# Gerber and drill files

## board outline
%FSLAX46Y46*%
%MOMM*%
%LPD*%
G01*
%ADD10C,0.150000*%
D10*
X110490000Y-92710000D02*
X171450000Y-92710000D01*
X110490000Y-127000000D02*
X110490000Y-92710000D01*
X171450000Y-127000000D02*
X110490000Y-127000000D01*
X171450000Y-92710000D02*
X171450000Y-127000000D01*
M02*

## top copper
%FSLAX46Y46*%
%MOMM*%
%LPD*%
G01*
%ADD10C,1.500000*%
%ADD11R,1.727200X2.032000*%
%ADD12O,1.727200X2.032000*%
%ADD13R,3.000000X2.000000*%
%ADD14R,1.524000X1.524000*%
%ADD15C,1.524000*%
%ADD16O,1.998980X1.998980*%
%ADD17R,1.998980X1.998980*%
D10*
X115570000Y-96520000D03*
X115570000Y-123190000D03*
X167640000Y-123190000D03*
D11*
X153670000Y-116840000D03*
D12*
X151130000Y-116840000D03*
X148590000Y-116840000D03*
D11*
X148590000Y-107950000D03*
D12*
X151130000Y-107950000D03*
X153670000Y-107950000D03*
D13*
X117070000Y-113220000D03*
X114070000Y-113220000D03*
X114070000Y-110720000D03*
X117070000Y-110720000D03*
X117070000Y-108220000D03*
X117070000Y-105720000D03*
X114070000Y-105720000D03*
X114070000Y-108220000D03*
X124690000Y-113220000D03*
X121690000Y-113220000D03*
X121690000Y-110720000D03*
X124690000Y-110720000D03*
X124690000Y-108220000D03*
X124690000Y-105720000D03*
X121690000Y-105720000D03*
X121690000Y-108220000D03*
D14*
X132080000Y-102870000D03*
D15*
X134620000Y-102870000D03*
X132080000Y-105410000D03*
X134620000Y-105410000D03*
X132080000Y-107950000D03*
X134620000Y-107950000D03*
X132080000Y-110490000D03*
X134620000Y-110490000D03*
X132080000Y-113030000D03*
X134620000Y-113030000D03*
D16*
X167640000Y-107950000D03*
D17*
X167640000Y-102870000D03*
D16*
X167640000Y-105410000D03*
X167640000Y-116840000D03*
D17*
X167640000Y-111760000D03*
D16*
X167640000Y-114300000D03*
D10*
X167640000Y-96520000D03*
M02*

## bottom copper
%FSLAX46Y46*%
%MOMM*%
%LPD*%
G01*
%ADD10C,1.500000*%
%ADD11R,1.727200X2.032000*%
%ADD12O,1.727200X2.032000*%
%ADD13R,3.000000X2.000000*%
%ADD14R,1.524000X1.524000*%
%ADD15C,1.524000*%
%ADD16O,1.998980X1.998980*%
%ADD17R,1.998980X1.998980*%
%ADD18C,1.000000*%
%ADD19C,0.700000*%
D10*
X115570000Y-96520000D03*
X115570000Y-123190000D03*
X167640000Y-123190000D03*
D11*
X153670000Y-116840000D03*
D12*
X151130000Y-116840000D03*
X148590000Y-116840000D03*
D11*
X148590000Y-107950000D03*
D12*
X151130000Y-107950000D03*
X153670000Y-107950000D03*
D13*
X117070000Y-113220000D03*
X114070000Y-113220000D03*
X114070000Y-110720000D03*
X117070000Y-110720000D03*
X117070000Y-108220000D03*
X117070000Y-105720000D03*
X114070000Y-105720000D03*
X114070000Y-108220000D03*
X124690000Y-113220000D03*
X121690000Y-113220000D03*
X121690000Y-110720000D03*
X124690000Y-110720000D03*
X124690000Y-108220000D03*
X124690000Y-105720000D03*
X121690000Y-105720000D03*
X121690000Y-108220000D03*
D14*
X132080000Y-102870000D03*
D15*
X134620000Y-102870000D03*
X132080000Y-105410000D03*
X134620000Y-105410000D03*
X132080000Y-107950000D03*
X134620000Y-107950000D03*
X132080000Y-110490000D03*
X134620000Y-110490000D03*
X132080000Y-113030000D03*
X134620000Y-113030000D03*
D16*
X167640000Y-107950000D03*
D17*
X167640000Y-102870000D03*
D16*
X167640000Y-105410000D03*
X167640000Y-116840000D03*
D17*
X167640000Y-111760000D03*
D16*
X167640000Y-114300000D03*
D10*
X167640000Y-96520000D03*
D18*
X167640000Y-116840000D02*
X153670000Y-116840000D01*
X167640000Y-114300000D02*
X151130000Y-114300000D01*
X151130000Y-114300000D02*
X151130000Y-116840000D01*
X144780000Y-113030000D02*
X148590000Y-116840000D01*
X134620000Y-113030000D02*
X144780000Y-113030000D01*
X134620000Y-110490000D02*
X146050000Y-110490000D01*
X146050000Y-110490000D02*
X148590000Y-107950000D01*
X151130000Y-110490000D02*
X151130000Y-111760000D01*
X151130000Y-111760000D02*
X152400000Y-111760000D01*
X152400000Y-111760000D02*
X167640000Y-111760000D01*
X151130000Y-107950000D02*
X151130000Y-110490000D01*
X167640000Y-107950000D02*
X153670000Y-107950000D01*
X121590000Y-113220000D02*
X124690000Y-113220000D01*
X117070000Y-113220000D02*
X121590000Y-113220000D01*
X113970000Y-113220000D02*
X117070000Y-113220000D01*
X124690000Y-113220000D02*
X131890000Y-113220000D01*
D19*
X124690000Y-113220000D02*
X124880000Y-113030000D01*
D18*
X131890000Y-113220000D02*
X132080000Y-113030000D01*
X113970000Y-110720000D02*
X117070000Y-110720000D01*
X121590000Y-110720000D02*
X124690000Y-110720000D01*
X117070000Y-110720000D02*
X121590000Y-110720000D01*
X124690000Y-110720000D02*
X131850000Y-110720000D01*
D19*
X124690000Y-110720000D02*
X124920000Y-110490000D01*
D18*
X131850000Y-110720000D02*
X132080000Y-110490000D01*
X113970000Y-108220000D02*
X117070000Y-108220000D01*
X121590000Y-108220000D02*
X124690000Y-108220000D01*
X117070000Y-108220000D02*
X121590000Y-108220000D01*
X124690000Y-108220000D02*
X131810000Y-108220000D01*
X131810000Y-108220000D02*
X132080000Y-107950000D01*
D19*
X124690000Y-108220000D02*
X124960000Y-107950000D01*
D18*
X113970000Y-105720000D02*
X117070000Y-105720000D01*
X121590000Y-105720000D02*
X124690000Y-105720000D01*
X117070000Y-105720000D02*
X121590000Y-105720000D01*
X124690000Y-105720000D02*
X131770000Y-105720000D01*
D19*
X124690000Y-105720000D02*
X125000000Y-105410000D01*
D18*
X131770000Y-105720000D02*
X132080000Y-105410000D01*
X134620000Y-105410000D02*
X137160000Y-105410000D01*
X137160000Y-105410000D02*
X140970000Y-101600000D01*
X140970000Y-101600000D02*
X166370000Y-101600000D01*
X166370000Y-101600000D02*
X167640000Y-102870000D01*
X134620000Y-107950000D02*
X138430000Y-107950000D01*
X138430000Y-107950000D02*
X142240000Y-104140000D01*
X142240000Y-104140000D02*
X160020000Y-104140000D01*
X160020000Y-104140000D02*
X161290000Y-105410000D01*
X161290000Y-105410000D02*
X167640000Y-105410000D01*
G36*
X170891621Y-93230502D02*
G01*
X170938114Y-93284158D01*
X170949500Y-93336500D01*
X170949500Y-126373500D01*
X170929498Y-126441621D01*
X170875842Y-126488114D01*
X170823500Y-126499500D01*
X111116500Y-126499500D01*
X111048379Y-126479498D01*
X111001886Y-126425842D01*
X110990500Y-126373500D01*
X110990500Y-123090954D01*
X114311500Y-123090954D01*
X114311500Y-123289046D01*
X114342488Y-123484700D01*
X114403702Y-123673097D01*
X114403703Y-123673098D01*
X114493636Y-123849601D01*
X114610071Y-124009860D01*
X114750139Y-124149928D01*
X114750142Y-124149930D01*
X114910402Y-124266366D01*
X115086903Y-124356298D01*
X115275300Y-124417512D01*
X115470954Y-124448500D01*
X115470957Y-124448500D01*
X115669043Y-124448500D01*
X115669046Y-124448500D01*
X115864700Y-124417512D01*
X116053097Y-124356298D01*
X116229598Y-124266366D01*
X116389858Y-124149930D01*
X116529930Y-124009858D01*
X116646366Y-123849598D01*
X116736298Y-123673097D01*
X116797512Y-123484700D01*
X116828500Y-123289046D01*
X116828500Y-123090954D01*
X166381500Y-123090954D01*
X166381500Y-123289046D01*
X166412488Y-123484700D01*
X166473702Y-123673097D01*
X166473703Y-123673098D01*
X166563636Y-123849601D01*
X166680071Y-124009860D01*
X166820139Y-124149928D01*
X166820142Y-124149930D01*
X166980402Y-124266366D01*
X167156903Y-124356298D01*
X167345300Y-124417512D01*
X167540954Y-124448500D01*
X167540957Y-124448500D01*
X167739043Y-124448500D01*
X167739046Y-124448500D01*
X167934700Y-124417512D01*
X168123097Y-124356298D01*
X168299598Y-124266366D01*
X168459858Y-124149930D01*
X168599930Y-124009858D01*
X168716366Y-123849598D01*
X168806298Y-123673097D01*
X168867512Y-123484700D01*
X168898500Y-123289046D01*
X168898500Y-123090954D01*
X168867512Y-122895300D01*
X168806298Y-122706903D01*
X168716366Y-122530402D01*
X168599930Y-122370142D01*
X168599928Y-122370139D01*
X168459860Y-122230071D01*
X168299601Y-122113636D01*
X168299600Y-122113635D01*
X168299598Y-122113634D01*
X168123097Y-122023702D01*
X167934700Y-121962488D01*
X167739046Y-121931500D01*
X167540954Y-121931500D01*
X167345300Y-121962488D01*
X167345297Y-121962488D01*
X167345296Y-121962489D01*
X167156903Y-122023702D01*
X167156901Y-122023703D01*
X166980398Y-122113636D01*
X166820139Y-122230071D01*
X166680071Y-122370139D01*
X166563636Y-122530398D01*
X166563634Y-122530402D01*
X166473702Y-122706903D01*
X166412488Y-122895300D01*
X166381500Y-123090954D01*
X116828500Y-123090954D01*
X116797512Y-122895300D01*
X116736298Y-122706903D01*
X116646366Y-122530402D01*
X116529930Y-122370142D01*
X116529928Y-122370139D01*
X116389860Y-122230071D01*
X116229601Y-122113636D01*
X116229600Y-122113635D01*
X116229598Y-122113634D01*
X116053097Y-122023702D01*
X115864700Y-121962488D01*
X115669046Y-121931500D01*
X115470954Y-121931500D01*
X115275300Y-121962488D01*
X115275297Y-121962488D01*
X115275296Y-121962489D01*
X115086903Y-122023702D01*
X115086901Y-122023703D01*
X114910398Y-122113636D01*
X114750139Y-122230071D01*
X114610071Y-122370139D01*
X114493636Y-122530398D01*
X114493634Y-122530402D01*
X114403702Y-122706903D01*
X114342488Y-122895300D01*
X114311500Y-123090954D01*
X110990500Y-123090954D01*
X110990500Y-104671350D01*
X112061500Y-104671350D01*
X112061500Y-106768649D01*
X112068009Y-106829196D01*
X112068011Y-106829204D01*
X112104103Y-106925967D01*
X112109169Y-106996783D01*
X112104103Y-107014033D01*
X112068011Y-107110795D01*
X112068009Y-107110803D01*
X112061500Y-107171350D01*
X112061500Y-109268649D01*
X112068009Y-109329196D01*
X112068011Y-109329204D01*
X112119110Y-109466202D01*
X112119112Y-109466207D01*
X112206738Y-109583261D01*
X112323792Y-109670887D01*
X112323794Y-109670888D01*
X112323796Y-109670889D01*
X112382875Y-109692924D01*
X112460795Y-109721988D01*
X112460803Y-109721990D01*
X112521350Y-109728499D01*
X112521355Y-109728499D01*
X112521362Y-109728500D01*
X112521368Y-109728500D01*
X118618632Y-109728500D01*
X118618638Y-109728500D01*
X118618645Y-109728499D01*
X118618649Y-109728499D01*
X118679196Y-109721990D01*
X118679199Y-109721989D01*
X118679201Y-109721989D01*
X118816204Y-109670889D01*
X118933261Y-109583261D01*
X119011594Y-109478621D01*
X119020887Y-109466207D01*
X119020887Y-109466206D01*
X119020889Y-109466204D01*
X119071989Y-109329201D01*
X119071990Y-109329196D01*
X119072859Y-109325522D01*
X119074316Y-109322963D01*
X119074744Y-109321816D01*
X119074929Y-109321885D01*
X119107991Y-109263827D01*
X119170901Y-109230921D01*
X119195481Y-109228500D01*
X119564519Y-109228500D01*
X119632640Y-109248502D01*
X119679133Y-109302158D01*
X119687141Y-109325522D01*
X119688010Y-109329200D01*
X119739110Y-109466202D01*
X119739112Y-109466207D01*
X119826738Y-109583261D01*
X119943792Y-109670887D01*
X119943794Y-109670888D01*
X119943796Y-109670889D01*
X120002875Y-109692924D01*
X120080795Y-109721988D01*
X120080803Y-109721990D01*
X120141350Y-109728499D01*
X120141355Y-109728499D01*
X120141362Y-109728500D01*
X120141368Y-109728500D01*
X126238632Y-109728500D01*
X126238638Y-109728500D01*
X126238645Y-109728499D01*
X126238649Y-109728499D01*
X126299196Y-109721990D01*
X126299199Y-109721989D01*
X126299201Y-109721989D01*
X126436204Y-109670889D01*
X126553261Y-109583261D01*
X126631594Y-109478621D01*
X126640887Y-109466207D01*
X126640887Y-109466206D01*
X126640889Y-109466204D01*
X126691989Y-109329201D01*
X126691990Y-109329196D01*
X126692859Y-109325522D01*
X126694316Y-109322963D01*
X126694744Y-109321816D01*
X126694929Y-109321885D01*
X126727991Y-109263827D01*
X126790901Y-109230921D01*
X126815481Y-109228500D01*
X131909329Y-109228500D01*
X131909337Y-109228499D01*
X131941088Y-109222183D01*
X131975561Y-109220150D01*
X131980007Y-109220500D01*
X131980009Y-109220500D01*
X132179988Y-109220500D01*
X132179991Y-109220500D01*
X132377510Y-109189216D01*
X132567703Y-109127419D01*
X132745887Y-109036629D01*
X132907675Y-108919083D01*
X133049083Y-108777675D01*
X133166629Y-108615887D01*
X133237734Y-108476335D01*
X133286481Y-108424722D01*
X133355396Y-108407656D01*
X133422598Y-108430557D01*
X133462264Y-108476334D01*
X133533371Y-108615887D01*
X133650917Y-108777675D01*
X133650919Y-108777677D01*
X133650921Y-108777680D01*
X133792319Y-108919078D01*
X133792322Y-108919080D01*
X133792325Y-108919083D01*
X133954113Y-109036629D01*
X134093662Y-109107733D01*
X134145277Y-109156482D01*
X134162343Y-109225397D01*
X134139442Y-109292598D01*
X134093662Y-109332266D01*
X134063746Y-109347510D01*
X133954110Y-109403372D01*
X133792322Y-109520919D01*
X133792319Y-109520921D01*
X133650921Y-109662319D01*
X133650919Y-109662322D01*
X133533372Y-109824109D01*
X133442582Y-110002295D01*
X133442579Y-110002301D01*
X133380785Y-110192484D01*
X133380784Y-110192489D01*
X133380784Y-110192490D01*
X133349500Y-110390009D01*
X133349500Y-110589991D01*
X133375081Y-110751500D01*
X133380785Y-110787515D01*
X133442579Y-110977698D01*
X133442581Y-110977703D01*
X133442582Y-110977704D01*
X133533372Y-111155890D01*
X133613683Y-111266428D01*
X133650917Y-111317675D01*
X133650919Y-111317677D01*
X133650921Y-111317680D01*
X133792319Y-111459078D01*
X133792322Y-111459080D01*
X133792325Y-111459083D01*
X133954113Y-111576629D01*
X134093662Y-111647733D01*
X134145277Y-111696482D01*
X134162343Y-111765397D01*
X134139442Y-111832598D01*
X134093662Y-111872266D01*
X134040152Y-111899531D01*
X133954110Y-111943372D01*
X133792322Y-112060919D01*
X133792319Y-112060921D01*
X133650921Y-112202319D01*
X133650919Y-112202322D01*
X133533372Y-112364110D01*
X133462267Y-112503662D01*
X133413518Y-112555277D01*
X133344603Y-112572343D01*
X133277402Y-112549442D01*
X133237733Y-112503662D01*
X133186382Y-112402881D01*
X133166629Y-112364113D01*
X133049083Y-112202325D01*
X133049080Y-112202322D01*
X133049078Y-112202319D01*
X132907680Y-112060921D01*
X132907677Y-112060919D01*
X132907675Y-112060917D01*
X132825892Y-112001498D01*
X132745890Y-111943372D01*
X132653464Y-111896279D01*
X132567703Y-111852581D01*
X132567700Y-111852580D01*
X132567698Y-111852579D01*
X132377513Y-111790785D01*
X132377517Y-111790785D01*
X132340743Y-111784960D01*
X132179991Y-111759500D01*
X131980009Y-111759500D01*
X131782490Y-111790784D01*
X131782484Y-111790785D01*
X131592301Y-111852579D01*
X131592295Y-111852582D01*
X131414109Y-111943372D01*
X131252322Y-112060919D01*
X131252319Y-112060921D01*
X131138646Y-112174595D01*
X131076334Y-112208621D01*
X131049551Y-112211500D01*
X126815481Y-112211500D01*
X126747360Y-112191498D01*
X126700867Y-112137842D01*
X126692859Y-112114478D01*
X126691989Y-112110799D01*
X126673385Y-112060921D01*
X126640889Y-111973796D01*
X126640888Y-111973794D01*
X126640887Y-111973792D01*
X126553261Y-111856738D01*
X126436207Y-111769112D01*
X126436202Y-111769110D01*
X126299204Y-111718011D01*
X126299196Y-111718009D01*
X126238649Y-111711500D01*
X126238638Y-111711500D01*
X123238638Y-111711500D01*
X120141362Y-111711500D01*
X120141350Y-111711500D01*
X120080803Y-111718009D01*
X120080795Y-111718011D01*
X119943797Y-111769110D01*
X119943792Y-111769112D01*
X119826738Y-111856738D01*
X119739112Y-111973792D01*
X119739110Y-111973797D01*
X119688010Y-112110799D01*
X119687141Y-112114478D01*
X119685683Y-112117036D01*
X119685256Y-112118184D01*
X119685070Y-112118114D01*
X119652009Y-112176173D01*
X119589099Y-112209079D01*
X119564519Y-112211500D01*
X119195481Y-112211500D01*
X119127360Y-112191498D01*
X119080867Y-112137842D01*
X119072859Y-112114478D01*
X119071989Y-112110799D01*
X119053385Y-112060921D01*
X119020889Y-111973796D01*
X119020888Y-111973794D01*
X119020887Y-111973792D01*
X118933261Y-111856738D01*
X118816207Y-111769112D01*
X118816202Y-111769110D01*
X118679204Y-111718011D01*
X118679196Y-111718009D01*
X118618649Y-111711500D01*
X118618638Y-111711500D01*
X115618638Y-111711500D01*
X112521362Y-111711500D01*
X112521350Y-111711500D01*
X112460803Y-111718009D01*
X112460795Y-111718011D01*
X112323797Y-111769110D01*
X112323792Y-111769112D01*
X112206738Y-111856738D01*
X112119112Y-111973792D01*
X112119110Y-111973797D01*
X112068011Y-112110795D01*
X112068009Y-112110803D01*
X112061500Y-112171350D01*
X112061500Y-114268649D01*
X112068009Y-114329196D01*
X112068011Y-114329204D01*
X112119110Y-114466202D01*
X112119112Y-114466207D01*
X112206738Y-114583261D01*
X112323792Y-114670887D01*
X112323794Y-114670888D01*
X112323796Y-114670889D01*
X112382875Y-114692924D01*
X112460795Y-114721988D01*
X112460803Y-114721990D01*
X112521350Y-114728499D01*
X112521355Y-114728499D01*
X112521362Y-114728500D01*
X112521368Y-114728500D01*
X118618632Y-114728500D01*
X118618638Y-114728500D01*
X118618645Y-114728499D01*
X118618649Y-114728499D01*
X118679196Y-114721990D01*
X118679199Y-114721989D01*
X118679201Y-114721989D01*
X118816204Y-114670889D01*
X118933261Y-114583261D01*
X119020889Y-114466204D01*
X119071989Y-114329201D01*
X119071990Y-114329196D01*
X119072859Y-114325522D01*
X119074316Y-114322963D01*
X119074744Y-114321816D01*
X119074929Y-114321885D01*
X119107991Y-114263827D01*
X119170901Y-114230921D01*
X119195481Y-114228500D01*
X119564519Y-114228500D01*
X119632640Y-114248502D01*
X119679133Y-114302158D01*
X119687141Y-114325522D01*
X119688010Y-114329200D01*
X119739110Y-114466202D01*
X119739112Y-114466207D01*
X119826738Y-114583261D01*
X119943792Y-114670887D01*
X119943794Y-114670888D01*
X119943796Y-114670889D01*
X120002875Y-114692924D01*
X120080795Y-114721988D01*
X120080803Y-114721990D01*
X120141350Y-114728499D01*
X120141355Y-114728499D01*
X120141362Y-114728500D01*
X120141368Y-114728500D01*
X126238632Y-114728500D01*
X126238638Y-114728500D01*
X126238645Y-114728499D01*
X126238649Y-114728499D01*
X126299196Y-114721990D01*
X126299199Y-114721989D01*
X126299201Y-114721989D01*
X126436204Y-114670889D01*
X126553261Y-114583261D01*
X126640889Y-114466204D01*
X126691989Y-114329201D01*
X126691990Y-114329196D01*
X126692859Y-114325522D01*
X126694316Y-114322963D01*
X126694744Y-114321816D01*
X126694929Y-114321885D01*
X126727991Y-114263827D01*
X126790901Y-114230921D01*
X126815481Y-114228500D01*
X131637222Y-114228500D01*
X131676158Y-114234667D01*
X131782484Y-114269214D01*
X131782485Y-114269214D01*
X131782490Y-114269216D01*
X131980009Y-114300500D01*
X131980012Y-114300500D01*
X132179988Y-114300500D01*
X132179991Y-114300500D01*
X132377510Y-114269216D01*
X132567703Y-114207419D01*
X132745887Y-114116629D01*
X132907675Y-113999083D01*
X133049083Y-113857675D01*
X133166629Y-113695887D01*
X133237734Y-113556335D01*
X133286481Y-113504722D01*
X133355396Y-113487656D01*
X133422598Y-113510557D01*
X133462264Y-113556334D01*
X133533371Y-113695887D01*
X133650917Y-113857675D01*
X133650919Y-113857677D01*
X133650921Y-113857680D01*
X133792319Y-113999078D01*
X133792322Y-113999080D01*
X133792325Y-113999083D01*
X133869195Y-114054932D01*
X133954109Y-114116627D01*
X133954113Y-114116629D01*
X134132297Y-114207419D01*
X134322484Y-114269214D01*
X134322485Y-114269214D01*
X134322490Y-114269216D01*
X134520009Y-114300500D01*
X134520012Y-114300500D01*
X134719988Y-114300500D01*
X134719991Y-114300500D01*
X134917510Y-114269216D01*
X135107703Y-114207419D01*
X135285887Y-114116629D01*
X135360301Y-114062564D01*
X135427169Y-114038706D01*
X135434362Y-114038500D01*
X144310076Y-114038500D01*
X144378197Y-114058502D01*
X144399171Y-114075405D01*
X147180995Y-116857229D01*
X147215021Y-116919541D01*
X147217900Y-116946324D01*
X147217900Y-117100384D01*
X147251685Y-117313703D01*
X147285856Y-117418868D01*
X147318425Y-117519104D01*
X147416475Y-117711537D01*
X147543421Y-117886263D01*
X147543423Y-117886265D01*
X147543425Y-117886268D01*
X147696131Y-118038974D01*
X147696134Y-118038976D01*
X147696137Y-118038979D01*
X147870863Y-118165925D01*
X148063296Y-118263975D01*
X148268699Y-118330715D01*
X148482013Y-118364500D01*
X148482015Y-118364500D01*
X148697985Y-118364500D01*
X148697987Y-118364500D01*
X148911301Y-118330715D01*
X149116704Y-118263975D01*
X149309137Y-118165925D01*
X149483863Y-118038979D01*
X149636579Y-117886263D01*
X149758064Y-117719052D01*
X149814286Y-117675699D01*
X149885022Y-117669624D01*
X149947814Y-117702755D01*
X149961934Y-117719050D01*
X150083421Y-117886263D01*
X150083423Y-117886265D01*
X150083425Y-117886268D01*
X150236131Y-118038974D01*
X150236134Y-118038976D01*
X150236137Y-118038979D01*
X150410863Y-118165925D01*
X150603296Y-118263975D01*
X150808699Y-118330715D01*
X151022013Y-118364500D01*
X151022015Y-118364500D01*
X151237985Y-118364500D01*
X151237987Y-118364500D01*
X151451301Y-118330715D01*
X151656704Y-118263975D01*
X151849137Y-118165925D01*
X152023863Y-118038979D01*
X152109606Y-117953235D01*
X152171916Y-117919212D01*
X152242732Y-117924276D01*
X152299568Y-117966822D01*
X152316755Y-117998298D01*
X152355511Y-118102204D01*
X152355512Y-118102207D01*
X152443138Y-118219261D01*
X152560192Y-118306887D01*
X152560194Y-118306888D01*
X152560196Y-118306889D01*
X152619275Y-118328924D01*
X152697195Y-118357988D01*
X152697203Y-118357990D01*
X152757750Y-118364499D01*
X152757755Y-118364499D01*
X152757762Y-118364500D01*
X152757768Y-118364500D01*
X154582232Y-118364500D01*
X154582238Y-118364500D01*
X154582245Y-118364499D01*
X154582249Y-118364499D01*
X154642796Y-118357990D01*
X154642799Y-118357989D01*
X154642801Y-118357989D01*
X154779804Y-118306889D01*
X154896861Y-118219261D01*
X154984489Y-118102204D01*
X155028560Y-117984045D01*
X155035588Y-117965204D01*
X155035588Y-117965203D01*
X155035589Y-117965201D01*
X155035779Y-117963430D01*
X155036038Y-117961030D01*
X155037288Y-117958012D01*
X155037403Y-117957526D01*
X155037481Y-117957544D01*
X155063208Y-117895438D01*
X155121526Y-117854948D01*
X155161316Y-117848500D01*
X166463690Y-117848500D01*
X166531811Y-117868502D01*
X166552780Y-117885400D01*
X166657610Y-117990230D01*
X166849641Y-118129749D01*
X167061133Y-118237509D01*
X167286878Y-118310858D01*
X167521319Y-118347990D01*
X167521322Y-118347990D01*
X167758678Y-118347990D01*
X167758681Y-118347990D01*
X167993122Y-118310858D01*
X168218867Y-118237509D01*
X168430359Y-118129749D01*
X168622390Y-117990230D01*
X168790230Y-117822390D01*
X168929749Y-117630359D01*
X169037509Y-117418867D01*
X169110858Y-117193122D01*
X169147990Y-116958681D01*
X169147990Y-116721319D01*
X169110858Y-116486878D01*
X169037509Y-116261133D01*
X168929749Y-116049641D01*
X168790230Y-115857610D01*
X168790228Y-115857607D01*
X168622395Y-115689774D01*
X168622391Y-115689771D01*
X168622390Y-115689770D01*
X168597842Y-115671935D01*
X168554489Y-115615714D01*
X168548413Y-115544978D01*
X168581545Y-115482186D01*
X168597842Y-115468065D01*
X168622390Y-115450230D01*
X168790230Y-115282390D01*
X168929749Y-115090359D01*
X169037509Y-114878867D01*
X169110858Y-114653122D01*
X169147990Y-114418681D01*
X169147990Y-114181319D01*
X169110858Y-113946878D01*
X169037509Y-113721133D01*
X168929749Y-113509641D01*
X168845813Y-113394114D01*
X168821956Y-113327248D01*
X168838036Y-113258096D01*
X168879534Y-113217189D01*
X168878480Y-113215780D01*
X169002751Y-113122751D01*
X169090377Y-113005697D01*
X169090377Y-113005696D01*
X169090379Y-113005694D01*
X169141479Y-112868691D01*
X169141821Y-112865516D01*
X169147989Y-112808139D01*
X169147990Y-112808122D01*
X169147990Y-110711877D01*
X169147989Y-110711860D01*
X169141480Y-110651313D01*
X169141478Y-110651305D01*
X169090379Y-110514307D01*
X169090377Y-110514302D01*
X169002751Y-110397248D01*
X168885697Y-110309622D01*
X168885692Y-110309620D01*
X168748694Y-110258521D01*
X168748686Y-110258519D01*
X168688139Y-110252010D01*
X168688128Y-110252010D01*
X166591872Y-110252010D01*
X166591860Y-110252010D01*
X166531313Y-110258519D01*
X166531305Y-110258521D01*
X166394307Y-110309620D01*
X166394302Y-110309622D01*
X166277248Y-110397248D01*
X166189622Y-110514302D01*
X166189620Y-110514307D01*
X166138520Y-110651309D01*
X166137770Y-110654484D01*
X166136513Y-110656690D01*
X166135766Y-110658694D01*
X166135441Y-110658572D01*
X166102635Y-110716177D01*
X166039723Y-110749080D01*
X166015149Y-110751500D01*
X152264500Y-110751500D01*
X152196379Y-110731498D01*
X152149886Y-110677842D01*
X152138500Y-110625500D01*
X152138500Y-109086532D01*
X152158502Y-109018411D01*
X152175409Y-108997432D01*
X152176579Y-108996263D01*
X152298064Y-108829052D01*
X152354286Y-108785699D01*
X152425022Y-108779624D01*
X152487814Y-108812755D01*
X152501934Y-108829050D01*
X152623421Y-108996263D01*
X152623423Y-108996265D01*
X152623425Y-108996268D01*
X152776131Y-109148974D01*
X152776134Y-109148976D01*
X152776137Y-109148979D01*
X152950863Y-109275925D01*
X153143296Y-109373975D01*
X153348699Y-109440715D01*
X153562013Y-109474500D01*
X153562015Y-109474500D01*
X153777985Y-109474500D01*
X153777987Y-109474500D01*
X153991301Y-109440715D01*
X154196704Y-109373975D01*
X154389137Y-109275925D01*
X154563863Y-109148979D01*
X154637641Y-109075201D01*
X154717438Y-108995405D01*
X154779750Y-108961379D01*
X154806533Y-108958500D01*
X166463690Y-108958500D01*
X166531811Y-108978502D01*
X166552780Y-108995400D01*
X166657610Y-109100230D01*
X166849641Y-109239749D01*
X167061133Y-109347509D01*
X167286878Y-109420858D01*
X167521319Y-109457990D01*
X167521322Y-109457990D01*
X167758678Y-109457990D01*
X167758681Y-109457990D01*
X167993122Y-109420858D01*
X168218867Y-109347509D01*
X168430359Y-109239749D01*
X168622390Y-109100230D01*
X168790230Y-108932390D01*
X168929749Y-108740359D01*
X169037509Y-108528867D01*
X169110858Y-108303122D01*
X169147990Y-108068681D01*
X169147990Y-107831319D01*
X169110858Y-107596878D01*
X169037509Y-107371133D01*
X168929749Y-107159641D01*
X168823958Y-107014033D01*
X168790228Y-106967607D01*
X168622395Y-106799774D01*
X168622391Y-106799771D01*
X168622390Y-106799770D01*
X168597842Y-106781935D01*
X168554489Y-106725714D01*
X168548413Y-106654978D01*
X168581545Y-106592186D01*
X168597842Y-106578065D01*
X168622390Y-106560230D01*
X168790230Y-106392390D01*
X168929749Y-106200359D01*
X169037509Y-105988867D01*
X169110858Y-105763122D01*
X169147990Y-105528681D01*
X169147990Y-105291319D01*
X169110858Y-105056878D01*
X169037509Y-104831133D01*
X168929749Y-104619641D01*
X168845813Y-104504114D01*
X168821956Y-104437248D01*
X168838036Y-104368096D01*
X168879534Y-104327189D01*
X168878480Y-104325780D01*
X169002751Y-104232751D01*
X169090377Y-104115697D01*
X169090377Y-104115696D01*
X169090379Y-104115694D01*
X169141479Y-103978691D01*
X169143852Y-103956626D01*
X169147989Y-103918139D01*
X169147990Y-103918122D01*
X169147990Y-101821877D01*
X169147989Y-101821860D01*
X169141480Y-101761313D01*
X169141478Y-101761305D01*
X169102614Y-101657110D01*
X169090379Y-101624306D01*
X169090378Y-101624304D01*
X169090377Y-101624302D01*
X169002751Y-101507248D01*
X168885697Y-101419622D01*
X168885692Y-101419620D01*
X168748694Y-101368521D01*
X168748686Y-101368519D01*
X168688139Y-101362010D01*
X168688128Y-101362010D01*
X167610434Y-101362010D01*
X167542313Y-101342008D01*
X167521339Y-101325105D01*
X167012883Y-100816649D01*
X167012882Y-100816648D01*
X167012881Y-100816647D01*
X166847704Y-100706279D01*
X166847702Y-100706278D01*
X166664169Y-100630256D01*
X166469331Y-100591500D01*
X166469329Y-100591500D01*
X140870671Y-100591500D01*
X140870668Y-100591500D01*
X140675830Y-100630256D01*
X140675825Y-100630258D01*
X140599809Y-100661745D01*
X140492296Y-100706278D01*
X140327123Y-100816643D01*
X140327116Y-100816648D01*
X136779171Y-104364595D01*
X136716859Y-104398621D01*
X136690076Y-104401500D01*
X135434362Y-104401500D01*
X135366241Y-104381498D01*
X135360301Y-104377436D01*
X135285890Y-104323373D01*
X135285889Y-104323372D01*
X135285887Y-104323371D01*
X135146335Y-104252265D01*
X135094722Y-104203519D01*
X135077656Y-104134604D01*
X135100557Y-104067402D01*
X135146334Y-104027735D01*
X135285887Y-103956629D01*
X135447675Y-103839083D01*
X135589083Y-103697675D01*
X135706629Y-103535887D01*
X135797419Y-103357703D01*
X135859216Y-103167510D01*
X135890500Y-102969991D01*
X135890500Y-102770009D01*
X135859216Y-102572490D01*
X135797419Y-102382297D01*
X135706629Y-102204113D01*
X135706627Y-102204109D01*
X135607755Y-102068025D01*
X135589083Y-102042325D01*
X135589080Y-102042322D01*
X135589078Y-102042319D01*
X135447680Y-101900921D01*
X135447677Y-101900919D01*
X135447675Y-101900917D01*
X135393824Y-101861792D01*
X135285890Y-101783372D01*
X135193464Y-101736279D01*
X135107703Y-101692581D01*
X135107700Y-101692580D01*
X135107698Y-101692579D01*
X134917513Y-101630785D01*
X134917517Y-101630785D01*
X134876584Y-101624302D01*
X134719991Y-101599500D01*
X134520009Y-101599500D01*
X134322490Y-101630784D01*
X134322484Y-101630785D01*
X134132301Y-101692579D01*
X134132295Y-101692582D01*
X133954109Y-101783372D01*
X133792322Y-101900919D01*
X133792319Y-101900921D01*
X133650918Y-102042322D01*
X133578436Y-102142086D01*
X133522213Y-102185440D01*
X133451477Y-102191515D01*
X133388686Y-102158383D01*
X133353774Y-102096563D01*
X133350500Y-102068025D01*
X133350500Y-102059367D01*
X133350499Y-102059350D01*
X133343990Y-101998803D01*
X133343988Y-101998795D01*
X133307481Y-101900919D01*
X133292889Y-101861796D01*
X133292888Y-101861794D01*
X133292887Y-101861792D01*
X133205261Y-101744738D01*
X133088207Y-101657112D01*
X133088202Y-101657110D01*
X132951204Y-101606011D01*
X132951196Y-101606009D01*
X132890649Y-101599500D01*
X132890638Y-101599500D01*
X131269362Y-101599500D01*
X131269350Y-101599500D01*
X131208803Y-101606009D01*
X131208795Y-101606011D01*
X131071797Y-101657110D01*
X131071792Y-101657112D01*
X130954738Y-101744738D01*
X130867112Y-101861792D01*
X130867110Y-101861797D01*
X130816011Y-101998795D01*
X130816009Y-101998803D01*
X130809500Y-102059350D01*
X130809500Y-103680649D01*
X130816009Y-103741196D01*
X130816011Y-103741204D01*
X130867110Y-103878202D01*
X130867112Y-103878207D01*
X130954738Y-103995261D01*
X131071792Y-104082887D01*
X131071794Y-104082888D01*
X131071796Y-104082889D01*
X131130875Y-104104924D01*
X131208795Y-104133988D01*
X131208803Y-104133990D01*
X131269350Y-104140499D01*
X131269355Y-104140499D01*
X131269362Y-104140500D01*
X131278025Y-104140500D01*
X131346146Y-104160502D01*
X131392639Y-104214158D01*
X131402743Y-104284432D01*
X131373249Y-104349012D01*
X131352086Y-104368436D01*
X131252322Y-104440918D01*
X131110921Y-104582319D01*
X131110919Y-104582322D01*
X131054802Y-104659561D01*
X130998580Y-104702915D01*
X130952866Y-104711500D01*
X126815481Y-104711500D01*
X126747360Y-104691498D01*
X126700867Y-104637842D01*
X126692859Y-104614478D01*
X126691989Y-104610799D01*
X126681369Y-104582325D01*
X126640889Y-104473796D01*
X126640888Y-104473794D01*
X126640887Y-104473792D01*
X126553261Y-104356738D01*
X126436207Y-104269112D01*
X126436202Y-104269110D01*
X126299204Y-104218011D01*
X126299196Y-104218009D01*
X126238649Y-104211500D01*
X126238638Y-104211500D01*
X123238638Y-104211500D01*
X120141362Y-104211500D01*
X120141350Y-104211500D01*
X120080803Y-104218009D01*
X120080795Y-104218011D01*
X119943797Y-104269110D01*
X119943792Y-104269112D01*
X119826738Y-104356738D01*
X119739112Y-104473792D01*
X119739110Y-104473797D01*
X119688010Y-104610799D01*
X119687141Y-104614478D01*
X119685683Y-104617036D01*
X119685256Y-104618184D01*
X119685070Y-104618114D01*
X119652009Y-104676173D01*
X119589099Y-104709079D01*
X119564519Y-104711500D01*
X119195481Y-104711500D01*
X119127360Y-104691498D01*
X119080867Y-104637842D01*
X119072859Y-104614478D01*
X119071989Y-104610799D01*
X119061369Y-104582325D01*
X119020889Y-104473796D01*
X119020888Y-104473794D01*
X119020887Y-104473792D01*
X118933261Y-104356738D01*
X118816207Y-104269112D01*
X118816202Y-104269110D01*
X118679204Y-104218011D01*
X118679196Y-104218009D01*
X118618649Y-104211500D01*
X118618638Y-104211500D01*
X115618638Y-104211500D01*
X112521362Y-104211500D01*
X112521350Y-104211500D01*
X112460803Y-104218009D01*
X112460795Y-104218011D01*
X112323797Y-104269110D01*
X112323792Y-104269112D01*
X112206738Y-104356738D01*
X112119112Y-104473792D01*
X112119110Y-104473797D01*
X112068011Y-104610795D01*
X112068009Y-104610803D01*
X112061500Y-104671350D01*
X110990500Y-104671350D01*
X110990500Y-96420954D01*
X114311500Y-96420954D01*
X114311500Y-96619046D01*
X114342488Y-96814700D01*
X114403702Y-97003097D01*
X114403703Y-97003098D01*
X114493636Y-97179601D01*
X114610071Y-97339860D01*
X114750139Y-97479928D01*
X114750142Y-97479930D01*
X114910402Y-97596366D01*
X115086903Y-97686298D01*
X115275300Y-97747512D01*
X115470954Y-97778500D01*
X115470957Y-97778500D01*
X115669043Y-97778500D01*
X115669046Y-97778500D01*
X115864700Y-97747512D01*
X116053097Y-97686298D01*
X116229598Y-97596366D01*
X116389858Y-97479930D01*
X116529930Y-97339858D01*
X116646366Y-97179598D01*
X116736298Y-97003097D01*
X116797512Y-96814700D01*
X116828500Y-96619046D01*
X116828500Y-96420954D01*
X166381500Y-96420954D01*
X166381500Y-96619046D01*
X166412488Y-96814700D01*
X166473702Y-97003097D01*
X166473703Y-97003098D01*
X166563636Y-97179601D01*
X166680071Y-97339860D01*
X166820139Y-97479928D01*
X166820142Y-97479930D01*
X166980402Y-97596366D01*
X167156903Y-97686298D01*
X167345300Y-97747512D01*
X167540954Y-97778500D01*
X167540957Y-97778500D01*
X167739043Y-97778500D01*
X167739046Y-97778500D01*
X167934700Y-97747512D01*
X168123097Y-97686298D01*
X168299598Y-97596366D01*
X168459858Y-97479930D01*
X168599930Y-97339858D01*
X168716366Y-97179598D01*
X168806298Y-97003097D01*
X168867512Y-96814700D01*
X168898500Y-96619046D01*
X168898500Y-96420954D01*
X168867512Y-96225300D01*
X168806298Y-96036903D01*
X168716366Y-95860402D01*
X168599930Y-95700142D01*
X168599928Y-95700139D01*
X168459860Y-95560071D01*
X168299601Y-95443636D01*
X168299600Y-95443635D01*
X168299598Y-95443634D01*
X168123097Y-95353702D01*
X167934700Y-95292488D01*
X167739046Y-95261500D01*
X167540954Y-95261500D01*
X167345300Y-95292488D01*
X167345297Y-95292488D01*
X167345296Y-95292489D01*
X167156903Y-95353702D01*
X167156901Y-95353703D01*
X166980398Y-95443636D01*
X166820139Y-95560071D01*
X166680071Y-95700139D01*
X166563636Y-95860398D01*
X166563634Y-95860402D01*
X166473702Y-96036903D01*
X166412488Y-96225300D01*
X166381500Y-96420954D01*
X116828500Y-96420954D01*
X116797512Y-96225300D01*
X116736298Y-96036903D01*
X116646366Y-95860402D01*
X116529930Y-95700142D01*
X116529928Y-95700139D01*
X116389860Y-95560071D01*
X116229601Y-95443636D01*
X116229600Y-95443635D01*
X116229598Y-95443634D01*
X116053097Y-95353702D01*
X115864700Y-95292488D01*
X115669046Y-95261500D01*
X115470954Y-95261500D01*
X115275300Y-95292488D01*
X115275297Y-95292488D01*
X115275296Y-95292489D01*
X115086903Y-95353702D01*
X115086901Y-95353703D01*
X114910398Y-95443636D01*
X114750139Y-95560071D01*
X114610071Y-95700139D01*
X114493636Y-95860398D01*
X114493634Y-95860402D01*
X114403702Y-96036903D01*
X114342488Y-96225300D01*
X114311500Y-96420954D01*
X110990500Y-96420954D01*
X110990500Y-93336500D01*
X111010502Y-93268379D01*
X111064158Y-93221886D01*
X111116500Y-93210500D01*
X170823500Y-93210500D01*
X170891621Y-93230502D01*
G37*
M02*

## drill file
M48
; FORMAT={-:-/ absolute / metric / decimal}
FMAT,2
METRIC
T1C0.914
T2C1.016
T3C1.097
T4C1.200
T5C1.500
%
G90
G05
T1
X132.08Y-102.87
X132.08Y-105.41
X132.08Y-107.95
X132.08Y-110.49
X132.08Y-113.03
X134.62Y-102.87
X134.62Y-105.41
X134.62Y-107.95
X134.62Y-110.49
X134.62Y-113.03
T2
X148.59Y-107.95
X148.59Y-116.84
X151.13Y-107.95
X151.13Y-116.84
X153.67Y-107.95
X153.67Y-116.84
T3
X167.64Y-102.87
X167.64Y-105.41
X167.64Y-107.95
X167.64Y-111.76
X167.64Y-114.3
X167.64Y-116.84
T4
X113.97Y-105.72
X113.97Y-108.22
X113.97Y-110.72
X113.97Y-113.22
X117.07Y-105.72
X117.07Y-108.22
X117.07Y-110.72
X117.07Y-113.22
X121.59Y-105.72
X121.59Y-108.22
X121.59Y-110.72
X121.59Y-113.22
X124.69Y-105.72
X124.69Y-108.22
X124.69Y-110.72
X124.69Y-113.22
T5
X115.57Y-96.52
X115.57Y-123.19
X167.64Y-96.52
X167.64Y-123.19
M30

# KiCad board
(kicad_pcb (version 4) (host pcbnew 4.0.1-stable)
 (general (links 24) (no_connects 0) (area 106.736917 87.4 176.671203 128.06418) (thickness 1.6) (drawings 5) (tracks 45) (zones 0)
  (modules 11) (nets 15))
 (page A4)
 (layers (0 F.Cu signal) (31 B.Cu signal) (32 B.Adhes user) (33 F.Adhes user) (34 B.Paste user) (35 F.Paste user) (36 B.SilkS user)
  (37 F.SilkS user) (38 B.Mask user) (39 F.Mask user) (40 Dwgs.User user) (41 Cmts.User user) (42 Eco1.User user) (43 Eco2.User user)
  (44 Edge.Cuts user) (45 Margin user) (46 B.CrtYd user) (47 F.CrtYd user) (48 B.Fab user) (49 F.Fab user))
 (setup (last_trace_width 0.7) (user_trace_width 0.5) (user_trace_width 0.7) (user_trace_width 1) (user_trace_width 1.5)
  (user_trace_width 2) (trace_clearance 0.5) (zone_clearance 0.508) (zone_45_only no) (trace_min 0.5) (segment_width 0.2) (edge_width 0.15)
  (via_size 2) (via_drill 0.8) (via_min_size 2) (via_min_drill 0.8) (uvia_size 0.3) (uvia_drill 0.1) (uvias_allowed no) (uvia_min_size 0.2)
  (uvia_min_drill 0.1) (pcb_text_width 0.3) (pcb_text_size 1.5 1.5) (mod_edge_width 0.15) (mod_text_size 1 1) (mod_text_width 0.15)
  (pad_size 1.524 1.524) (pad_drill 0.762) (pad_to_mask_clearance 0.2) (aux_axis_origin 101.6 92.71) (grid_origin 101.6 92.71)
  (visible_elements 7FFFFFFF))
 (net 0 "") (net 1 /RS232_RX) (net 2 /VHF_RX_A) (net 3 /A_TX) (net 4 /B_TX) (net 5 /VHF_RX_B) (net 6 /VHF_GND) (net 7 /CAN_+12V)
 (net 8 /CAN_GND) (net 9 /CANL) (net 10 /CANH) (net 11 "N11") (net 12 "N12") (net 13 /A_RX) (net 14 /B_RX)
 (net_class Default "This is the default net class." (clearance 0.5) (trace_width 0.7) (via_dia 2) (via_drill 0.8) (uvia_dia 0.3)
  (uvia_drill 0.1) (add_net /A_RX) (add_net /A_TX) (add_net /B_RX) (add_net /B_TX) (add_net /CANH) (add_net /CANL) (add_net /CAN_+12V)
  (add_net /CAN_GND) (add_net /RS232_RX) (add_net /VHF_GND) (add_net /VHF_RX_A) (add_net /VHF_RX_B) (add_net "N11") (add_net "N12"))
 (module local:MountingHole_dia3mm (layer F.Cu) (at 115.57 96.52)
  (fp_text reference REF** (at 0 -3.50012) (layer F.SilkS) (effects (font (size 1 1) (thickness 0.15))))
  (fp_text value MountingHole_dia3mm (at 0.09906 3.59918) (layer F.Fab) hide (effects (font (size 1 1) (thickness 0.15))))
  (pad 1 thru_hole circle (at 0 0) (size 1.5 1.5) (drill 1.5) (layers *.Cu) (zone_connect 0)))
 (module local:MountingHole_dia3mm (layer F.Cu) (at 115.57 123.19)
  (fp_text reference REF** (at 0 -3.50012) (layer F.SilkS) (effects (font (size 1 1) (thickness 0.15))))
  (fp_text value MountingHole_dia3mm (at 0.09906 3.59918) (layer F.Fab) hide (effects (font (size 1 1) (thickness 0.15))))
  (pad 1 thru_hole circle (at 0 0) (size 1.5 1.5) (drill 1.5) (layers *.Cu) (zone_connect 0)))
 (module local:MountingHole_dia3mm (layer F.Cu) (at 167.64 123.19)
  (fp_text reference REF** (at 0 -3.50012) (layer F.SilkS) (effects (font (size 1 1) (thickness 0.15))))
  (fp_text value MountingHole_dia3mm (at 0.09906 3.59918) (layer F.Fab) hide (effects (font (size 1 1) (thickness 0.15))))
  (pad 1 thru_hole circle (at 0 0) (size 1.5 1.5) (drill 1.5) (layers *.Cu) (zone_connect 0)))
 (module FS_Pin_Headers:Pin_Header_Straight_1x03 (layer F.Cu) (at 153.67 116.84 270)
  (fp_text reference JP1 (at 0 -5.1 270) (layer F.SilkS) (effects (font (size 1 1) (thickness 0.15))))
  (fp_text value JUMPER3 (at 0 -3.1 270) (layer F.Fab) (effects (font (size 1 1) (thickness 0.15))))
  (pad 1 thru_hole rect (at 0 0 270) (size 2.032 1.7272) (drill 1.016) (layers *.Cu *.Mask F.SilkS) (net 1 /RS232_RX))
  (pad 2 thru_hole oval (at 0 2.54 270) (size 2.032 1.7272) (drill 1.016) (layers *.Cu *.Mask F.SilkS) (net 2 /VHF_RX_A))
  (pad 3 thru_hole oval (at 0 5.08 270) (size 2.032 1.7272) (drill 1.016) (layers *.Cu *.Mask F.SilkS) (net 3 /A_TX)))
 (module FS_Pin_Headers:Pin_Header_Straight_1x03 (layer F.Cu) (at 148.59 107.95 90)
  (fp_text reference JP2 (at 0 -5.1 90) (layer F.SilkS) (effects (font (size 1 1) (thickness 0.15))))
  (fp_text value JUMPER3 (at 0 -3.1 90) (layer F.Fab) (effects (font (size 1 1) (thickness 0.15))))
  (pad 1 thru_hole rect (at 0 0 90) (size 2.032 1.7272) (drill 1.016) (layers *.Cu *.Mask F.SilkS) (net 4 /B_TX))
  (pad 2 thru_hole oval (at 0 2.54 90) (size 2.032 1.7272) (drill 1.016) (layers *.Cu *.Mask F.SilkS) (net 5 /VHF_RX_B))
  (pad 3 thru_hole oval (at 0 5.08 90) (size 2.032 1.7272) (drill 1.016) (layers *.Cu *.Mask F.SilkS) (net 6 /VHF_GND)))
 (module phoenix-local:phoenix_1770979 (layer F.Cu) (at 115.57 109.22 90)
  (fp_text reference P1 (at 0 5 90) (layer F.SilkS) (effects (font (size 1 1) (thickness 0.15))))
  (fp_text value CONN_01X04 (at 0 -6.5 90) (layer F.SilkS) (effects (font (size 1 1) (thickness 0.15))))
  (pad 1 thru_hole rect (at -4 1.5 90) (size 2 3) (drill 1.2) (layers *.Cu *.Mask F.SilkS) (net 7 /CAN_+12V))
  (pad 1 thru_hole rect (at -4 -1.6 90) (size 2 3) (drill 1.2 (offset 0 0.1)) (layers *.Cu *.Mask F.SilkS) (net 7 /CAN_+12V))
  (pad 2 thru_hole rect (at -1.5 -1.6 90) (size 2 3) (drill 1.2 (offset 0 0.1)) (layers *.Cu *.Mask F.SilkS) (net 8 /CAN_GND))
  (pad 2 thru_hole rect (at -1.5 1.5 90) (size 2 3) (drill 1.2) (layers *.Cu *.Mask F.SilkS) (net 8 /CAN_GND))
  (pad 3 thru_hole rect (at 1 1.5 90) (size 2 3) (drill 1.2) (layers *.Cu *.Mask F.SilkS) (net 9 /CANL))
  (pad 4 thru_hole rect (at 3.5 1.5 90) (size 2 3) (drill 1.2) (layers *.Cu *.Mask F.SilkS) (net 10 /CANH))
  (pad 4 thru_hole rect (at 3.5 -1.6 90) (size 2 3) (drill 1.2 (offset 0 0.1)) (layers *.Cu *.Mask F.SilkS) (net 10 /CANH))
  (pad 3 thru_hole rect (at 1 -1.6 90) (size 2 3) (drill 1.2 (offset 0 0.1)) (layers *.Cu *.Mask F.SilkS) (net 9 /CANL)))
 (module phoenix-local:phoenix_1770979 (layer F.Cu) (at 123.19 109.22 90)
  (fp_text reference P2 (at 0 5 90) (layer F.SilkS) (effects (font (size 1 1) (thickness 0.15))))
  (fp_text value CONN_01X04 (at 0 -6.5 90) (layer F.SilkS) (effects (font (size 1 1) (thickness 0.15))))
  (pad 1 thru_hole rect (at -4 1.5 90) (size 2 3) (drill 1.2) (layers *.Cu *.Mask F.SilkS) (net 7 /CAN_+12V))
  (pad 1 thru_hole rect (at -4 -1.6 90) (size 2 3) (drill 1.2 (offset 0 0.1)) (layers *.Cu *.Mask F.SilkS) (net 7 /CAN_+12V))
  (pad 2 thru_hole rect (at -1.5 -1.6 90) (size 2 3) (drill 1.2 (offset 0 0.1)) (layers *.Cu *.Mask F.SilkS) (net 8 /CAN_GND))
  (pad 2 thru_hole rect (at -1.5 1.5 90) (size 2 3) (drill 1.2) (layers *.Cu *.Mask F.SilkS) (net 8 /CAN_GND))
  (pad 3 thru_hole rect (at 1 1.5 90) (size 2 3) (drill 1.2) (layers *.Cu *.Mask F.SilkS) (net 9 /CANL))
  (pad 4 thru_hole rect (at 3.5 1.5 90) (size 2 3) (drill 1.2) (layers *.Cu *.Mask F.SilkS) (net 10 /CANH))
  (pad 4 thru_hole rect (at 3.5 -1.6 90) (size 2 3) (drill 1.2 (offset 0 0.1)) (layers *.Cu *.Mask F.SilkS) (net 10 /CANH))
  (pad 3 thru_hole rect (at 1 -1.6 90) (size 2 3) (drill 1.2 (offset 0 0.1)) (layers *.Cu *.Mask F.SilkS) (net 9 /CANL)))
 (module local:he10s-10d (layer F.Cu) (at 133.35 107.95 270)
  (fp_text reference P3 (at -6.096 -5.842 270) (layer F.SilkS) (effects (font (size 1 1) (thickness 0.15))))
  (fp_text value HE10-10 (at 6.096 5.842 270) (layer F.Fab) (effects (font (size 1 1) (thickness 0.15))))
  (pad 1 thru_hole rect (at -5.08 1.27 270) (size 1.524 1.524) (drill 0.9144) (layers *.Cu *.Mask F.SilkS) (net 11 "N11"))
  (pad 2 thru_hole circle (at -5.08 -1.27 270) (size 1.524 1.524) (drill 0.9144) (layers *.Cu *.Mask F.SilkS) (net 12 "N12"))
  (pad 3 thru_hole circle (at -2.54 1.27 270) (size 1.524 1.524) (drill 0.9144) (layers *.Cu *.Mask F.SilkS) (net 10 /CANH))
  (pad 4 thru_hole circle (at -2.54 -1.27 270) (size 1.524 1.524) (drill 0.9144) (layers *.Cu *.Mask F.SilkS) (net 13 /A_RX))
  (pad 5 thru_hole circle (at 0 1.27 270) (size 1.524 1.524) (drill 0.9144) (layers *.Cu *.Mask F.SilkS) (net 9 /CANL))
  (pad 6 thru_hole circle (at 0 -1.27 270) (size 1.524 1.524) (drill 0.9144) (layers *.Cu *.Mask F.SilkS) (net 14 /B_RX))
  (pad 7 thru_hole circle (at 2.54 1.27 270) (size 1.524 1.524) (drill 0.9144) (layers *.Cu *.Mask F.SilkS) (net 8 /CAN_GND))
  (pad 8 thru_hole circle (at 2.54 -1.27 270) (size 1.524 1.524) (drill 0.9144) (layers *.Cu *.Mask F.SilkS) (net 4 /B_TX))
  (pad 9 thru_hole circle (at 5.08 1.27 270) (size 1.524 1.524) (drill 0.9144) (layers *.Cu *.Mask F.SilkS) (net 7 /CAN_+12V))
  (pad 10 thru_hole circle (at 5.08 -1.27 270) (size 1.524 1.524) (drill 0.9144) (layers *.Cu *.Mask F.SilkS) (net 3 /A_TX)))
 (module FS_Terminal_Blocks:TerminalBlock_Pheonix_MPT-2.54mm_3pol (layer F.Cu) (at 167.64 102.87 270)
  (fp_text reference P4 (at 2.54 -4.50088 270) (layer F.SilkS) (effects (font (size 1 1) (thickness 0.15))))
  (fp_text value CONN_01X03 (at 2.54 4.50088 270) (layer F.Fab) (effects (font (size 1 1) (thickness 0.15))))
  (pad 3 thru_hole oval (at 5.08 0 270) (size 1.99898 1.99898) (drill 1.09728) (layers *.Cu *.Mask F.SilkS) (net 6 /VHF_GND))
  (pad 1 thru_hole rect (at 0 0 270) (size 1.99898 1.99898) (drill 1.09728) (layers *.Cu *.Mask F.SilkS) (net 13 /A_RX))
  (pad 2 thru_hole oval (at 2.54 0 270) (size 1.99898 1.99898) (drill 1.09728) (layers *.Cu *.Mask F.SilkS) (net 14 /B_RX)))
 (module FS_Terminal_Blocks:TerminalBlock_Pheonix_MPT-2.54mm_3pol (layer F.Cu) (at 167.64 111.76 270)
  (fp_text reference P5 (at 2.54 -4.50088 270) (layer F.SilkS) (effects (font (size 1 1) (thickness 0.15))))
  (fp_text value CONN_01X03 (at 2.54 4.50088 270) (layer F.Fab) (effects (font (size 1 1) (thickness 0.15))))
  (pad 3 thru_hole oval (at 5.08 0 270) (size 1.99898 1.99898) (drill 1.09728) (layers *.Cu *.Mask F.SilkS) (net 1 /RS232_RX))
  (pad 1 thru_hole rect (at 0 0 270) (size 1.99898 1.99898) (drill 1.09728) (layers *.Cu *.Mask F.SilkS) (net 5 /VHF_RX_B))
  (pad 2 thru_hole oval (at 2.54 0 270) (size 1.99898 1.99898) (drill 1.09728) (layers *.Cu *.Mask F.SilkS) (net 2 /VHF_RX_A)))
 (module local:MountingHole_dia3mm (layer F.Cu) (at 167.64 96.52)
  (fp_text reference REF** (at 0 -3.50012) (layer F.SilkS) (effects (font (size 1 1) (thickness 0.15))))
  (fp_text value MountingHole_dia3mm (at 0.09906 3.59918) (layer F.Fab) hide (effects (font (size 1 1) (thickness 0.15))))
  (pad 1 thru_hole circle (at 0 0) (size 1.5 1.5) (drill 1.5) (layers *.Cu) (zone_connect 0)))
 (gr_line (start 110.49 92.71) (end 171.45 92.71) (angle 90) (layer Edge.Cuts) (width 0.15))
 (gr_line (start 110.49 127) (end 110.49 92.71) (angle 90) (layer Edge.Cuts) (width 0.15))
 (gr_line (start 171.45 127) (end 110.49 127) (angle 90) (layer Edge.Cuts) (width 0.15))
 (gr_line (start 171.45 92.71) (end 171.45 127) (angle 90) (layer Edge.Cuts) (width 0.15))
 (segment (start 167.64 116.84) (end 153.67 116.84) (width 1) (layer B.Cu) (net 1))
 (segment (start 167.64 114.3) (end 151.13 114.3) (width 1) (layer B.Cu) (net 2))
 (segment (start 151.13 114.3) (end 151.13 116.84) (width 1) (layer B.Cu) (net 2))
 (segment (start 144.78 113.03) (end 148.59 116.84) (width 1) (layer B.Cu) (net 3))
 (segment (start 134.62 113.03) (end 144.78 113.03) (width 1) (layer B.Cu) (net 3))
 (segment (start 134.62 110.49) (end 146.05 110.49) (width 1) (layer B.Cu) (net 4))
 (segment (start 146.05 110.49) (end 148.59 107.95) (width 1) (layer B.Cu) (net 4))
 (segment (start 151.13 110.49) (end 151.13 111.76) (width 1) (layer B.Cu) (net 5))
 (segment (start 151.13 111.76) (end 152.4 111.76) (width 1) (layer B.Cu) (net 5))
 (segment (start 152.4 111.76) (end 167.64 111.76) (width 1) (layer B.Cu) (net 5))
 (segment (start 151.13 107.95) (end 151.13 110.49) (width 1) (layer B.Cu) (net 5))
 (segment (start 167.64 107.95) (end 153.67 107.95) (width 1) (layer B.Cu) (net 6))
 (segment (start 121.59 113.22) (end 124.69 113.22) (width 1) (layer B.Cu) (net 7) (status 30))
 (segment (start 117.07 113.22) (end 121.59 113.22) (width 1) (layer B.Cu) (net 7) (status 10))
 (segment (start 113.97 113.22) (end 117.07 113.22) (width 1) (layer B.Cu) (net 7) (status 30))
 (segment (start 124.69 113.22) (end 131.89 113.22) (width 1) (layer B.Cu) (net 7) (status 10))
 (segment (start 124.69 113.22) (end 124.88 113.03) (width 0.7) (layer B.Cu) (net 7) (status 30))
 (segment (start 131.89 113.22) (end 132.08 113.03) (width 1) (layer B.Cu) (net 7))
 (segment (start 113.97 110.72) (end 117.07 110.72) (width 1) (layer B.Cu) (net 8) (status 30))
 (segment (start 121.59 110.72) (end 124.69 110.72) (width 1) (layer B.Cu) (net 8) (status 30))
 (segment (start 117.07 110.72) (end 121.59 110.72) (width 1) (layer B.Cu) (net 8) (status 10))
 (segment (start 124.69 110.72) (end 131.85 110.72) (width 1) (layer B.Cu) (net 8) (status 10))
 (segment (start 124.69 110.72) (end 124.92 110.49) (width 0.7) (layer B.Cu) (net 8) (status 30))
 (segment (start 131.85 110.72) (end 132.08 110.49) (width 1) (layer B.Cu) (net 8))
 (segment (start 113.97 108.22) (end 117.07 108.22) (width 1) (layer B.Cu) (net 9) (status 30))
 (segment (start 121.59 108.22) (end 124.69 108.22) (width 1) (layer B.Cu) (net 9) (status 30))
 (segment (start 117.07 108.22) (end 121.59 108.22) (width 1) (layer B.Cu) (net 9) (status 10))
 (segment (start 124.69 108.22) (end 131.81 108.22) (width 1) (layer B.Cu) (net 9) (status 10))
 (segment (start 131.81 108.22) (end 132.08 107.95) (width 1) (layer B.Cu) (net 9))
 (segment (start 124.69 108.22) (end 124.96 107.95) (width 0.7) (layer B.Cu) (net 9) (status 30))
 (segment (start 113.97 105.72) (end 117.07 105.72) (width 1) (layer B.Cu) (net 10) (status 30))
 (segment (start 121.59 105.72) (end 124.69 105.72) (width 1) (layer B.Cu) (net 10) (status 30))
 (segment (start 117.07 105.72) (end 121.59 105.72) (width 1) (layer B.Cu) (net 10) (status 10))
 (segment (start 124.69 105.72) (end 131.77 105.72) (width 1) (layer B.Cu) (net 10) (status 10))
 (segment (start 124.69 105.72) (end 125 105.41) (width 0.7) (layer B.Cu) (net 10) (status 30))
 (segment (start 131.77 105.72) (end 132.08 105.41) (width 1) (layer B.Cu) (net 10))
 (segment (start 134.62 105.41) (end 137.16 105.41) (width 1) (layer B.Cu) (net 13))
 (segment (start 137.16 105.41) (end 140.97 101.6) (width 1) (layer B.Cu) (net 13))
 (segment (start 140.97 101.6) (end 166.37 101.6) (width 1) (layer B.Cu) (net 13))
 (segment (start 166.37 101.6) (end 167.64 102.87) (width 1) (layer B.Cu) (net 13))
 (segment (start 134.62 107.95) (end 138.43 107.95) (width 1) (layer B.Cu) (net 14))
 (segment (start 138.43 107.95) (end 142.24 104.14) (width 1) (layer B.Cu) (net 14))
 (segment (start 142.24 104.14) (end 160.02 104.14) (width 1) (layer B.Cu) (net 14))
 (segment (start 160.02 104.14) (end 161.29 105.41) (width 1) (layer B.Cu) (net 14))
 (segment (start 161.29 105.41) (end 167.64 105.41) (width 1) (layer B.Cu) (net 14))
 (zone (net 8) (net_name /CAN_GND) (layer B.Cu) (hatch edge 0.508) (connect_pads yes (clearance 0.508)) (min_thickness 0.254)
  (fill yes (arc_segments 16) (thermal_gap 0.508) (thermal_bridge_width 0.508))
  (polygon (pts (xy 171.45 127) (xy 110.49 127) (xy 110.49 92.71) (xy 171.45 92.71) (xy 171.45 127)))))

